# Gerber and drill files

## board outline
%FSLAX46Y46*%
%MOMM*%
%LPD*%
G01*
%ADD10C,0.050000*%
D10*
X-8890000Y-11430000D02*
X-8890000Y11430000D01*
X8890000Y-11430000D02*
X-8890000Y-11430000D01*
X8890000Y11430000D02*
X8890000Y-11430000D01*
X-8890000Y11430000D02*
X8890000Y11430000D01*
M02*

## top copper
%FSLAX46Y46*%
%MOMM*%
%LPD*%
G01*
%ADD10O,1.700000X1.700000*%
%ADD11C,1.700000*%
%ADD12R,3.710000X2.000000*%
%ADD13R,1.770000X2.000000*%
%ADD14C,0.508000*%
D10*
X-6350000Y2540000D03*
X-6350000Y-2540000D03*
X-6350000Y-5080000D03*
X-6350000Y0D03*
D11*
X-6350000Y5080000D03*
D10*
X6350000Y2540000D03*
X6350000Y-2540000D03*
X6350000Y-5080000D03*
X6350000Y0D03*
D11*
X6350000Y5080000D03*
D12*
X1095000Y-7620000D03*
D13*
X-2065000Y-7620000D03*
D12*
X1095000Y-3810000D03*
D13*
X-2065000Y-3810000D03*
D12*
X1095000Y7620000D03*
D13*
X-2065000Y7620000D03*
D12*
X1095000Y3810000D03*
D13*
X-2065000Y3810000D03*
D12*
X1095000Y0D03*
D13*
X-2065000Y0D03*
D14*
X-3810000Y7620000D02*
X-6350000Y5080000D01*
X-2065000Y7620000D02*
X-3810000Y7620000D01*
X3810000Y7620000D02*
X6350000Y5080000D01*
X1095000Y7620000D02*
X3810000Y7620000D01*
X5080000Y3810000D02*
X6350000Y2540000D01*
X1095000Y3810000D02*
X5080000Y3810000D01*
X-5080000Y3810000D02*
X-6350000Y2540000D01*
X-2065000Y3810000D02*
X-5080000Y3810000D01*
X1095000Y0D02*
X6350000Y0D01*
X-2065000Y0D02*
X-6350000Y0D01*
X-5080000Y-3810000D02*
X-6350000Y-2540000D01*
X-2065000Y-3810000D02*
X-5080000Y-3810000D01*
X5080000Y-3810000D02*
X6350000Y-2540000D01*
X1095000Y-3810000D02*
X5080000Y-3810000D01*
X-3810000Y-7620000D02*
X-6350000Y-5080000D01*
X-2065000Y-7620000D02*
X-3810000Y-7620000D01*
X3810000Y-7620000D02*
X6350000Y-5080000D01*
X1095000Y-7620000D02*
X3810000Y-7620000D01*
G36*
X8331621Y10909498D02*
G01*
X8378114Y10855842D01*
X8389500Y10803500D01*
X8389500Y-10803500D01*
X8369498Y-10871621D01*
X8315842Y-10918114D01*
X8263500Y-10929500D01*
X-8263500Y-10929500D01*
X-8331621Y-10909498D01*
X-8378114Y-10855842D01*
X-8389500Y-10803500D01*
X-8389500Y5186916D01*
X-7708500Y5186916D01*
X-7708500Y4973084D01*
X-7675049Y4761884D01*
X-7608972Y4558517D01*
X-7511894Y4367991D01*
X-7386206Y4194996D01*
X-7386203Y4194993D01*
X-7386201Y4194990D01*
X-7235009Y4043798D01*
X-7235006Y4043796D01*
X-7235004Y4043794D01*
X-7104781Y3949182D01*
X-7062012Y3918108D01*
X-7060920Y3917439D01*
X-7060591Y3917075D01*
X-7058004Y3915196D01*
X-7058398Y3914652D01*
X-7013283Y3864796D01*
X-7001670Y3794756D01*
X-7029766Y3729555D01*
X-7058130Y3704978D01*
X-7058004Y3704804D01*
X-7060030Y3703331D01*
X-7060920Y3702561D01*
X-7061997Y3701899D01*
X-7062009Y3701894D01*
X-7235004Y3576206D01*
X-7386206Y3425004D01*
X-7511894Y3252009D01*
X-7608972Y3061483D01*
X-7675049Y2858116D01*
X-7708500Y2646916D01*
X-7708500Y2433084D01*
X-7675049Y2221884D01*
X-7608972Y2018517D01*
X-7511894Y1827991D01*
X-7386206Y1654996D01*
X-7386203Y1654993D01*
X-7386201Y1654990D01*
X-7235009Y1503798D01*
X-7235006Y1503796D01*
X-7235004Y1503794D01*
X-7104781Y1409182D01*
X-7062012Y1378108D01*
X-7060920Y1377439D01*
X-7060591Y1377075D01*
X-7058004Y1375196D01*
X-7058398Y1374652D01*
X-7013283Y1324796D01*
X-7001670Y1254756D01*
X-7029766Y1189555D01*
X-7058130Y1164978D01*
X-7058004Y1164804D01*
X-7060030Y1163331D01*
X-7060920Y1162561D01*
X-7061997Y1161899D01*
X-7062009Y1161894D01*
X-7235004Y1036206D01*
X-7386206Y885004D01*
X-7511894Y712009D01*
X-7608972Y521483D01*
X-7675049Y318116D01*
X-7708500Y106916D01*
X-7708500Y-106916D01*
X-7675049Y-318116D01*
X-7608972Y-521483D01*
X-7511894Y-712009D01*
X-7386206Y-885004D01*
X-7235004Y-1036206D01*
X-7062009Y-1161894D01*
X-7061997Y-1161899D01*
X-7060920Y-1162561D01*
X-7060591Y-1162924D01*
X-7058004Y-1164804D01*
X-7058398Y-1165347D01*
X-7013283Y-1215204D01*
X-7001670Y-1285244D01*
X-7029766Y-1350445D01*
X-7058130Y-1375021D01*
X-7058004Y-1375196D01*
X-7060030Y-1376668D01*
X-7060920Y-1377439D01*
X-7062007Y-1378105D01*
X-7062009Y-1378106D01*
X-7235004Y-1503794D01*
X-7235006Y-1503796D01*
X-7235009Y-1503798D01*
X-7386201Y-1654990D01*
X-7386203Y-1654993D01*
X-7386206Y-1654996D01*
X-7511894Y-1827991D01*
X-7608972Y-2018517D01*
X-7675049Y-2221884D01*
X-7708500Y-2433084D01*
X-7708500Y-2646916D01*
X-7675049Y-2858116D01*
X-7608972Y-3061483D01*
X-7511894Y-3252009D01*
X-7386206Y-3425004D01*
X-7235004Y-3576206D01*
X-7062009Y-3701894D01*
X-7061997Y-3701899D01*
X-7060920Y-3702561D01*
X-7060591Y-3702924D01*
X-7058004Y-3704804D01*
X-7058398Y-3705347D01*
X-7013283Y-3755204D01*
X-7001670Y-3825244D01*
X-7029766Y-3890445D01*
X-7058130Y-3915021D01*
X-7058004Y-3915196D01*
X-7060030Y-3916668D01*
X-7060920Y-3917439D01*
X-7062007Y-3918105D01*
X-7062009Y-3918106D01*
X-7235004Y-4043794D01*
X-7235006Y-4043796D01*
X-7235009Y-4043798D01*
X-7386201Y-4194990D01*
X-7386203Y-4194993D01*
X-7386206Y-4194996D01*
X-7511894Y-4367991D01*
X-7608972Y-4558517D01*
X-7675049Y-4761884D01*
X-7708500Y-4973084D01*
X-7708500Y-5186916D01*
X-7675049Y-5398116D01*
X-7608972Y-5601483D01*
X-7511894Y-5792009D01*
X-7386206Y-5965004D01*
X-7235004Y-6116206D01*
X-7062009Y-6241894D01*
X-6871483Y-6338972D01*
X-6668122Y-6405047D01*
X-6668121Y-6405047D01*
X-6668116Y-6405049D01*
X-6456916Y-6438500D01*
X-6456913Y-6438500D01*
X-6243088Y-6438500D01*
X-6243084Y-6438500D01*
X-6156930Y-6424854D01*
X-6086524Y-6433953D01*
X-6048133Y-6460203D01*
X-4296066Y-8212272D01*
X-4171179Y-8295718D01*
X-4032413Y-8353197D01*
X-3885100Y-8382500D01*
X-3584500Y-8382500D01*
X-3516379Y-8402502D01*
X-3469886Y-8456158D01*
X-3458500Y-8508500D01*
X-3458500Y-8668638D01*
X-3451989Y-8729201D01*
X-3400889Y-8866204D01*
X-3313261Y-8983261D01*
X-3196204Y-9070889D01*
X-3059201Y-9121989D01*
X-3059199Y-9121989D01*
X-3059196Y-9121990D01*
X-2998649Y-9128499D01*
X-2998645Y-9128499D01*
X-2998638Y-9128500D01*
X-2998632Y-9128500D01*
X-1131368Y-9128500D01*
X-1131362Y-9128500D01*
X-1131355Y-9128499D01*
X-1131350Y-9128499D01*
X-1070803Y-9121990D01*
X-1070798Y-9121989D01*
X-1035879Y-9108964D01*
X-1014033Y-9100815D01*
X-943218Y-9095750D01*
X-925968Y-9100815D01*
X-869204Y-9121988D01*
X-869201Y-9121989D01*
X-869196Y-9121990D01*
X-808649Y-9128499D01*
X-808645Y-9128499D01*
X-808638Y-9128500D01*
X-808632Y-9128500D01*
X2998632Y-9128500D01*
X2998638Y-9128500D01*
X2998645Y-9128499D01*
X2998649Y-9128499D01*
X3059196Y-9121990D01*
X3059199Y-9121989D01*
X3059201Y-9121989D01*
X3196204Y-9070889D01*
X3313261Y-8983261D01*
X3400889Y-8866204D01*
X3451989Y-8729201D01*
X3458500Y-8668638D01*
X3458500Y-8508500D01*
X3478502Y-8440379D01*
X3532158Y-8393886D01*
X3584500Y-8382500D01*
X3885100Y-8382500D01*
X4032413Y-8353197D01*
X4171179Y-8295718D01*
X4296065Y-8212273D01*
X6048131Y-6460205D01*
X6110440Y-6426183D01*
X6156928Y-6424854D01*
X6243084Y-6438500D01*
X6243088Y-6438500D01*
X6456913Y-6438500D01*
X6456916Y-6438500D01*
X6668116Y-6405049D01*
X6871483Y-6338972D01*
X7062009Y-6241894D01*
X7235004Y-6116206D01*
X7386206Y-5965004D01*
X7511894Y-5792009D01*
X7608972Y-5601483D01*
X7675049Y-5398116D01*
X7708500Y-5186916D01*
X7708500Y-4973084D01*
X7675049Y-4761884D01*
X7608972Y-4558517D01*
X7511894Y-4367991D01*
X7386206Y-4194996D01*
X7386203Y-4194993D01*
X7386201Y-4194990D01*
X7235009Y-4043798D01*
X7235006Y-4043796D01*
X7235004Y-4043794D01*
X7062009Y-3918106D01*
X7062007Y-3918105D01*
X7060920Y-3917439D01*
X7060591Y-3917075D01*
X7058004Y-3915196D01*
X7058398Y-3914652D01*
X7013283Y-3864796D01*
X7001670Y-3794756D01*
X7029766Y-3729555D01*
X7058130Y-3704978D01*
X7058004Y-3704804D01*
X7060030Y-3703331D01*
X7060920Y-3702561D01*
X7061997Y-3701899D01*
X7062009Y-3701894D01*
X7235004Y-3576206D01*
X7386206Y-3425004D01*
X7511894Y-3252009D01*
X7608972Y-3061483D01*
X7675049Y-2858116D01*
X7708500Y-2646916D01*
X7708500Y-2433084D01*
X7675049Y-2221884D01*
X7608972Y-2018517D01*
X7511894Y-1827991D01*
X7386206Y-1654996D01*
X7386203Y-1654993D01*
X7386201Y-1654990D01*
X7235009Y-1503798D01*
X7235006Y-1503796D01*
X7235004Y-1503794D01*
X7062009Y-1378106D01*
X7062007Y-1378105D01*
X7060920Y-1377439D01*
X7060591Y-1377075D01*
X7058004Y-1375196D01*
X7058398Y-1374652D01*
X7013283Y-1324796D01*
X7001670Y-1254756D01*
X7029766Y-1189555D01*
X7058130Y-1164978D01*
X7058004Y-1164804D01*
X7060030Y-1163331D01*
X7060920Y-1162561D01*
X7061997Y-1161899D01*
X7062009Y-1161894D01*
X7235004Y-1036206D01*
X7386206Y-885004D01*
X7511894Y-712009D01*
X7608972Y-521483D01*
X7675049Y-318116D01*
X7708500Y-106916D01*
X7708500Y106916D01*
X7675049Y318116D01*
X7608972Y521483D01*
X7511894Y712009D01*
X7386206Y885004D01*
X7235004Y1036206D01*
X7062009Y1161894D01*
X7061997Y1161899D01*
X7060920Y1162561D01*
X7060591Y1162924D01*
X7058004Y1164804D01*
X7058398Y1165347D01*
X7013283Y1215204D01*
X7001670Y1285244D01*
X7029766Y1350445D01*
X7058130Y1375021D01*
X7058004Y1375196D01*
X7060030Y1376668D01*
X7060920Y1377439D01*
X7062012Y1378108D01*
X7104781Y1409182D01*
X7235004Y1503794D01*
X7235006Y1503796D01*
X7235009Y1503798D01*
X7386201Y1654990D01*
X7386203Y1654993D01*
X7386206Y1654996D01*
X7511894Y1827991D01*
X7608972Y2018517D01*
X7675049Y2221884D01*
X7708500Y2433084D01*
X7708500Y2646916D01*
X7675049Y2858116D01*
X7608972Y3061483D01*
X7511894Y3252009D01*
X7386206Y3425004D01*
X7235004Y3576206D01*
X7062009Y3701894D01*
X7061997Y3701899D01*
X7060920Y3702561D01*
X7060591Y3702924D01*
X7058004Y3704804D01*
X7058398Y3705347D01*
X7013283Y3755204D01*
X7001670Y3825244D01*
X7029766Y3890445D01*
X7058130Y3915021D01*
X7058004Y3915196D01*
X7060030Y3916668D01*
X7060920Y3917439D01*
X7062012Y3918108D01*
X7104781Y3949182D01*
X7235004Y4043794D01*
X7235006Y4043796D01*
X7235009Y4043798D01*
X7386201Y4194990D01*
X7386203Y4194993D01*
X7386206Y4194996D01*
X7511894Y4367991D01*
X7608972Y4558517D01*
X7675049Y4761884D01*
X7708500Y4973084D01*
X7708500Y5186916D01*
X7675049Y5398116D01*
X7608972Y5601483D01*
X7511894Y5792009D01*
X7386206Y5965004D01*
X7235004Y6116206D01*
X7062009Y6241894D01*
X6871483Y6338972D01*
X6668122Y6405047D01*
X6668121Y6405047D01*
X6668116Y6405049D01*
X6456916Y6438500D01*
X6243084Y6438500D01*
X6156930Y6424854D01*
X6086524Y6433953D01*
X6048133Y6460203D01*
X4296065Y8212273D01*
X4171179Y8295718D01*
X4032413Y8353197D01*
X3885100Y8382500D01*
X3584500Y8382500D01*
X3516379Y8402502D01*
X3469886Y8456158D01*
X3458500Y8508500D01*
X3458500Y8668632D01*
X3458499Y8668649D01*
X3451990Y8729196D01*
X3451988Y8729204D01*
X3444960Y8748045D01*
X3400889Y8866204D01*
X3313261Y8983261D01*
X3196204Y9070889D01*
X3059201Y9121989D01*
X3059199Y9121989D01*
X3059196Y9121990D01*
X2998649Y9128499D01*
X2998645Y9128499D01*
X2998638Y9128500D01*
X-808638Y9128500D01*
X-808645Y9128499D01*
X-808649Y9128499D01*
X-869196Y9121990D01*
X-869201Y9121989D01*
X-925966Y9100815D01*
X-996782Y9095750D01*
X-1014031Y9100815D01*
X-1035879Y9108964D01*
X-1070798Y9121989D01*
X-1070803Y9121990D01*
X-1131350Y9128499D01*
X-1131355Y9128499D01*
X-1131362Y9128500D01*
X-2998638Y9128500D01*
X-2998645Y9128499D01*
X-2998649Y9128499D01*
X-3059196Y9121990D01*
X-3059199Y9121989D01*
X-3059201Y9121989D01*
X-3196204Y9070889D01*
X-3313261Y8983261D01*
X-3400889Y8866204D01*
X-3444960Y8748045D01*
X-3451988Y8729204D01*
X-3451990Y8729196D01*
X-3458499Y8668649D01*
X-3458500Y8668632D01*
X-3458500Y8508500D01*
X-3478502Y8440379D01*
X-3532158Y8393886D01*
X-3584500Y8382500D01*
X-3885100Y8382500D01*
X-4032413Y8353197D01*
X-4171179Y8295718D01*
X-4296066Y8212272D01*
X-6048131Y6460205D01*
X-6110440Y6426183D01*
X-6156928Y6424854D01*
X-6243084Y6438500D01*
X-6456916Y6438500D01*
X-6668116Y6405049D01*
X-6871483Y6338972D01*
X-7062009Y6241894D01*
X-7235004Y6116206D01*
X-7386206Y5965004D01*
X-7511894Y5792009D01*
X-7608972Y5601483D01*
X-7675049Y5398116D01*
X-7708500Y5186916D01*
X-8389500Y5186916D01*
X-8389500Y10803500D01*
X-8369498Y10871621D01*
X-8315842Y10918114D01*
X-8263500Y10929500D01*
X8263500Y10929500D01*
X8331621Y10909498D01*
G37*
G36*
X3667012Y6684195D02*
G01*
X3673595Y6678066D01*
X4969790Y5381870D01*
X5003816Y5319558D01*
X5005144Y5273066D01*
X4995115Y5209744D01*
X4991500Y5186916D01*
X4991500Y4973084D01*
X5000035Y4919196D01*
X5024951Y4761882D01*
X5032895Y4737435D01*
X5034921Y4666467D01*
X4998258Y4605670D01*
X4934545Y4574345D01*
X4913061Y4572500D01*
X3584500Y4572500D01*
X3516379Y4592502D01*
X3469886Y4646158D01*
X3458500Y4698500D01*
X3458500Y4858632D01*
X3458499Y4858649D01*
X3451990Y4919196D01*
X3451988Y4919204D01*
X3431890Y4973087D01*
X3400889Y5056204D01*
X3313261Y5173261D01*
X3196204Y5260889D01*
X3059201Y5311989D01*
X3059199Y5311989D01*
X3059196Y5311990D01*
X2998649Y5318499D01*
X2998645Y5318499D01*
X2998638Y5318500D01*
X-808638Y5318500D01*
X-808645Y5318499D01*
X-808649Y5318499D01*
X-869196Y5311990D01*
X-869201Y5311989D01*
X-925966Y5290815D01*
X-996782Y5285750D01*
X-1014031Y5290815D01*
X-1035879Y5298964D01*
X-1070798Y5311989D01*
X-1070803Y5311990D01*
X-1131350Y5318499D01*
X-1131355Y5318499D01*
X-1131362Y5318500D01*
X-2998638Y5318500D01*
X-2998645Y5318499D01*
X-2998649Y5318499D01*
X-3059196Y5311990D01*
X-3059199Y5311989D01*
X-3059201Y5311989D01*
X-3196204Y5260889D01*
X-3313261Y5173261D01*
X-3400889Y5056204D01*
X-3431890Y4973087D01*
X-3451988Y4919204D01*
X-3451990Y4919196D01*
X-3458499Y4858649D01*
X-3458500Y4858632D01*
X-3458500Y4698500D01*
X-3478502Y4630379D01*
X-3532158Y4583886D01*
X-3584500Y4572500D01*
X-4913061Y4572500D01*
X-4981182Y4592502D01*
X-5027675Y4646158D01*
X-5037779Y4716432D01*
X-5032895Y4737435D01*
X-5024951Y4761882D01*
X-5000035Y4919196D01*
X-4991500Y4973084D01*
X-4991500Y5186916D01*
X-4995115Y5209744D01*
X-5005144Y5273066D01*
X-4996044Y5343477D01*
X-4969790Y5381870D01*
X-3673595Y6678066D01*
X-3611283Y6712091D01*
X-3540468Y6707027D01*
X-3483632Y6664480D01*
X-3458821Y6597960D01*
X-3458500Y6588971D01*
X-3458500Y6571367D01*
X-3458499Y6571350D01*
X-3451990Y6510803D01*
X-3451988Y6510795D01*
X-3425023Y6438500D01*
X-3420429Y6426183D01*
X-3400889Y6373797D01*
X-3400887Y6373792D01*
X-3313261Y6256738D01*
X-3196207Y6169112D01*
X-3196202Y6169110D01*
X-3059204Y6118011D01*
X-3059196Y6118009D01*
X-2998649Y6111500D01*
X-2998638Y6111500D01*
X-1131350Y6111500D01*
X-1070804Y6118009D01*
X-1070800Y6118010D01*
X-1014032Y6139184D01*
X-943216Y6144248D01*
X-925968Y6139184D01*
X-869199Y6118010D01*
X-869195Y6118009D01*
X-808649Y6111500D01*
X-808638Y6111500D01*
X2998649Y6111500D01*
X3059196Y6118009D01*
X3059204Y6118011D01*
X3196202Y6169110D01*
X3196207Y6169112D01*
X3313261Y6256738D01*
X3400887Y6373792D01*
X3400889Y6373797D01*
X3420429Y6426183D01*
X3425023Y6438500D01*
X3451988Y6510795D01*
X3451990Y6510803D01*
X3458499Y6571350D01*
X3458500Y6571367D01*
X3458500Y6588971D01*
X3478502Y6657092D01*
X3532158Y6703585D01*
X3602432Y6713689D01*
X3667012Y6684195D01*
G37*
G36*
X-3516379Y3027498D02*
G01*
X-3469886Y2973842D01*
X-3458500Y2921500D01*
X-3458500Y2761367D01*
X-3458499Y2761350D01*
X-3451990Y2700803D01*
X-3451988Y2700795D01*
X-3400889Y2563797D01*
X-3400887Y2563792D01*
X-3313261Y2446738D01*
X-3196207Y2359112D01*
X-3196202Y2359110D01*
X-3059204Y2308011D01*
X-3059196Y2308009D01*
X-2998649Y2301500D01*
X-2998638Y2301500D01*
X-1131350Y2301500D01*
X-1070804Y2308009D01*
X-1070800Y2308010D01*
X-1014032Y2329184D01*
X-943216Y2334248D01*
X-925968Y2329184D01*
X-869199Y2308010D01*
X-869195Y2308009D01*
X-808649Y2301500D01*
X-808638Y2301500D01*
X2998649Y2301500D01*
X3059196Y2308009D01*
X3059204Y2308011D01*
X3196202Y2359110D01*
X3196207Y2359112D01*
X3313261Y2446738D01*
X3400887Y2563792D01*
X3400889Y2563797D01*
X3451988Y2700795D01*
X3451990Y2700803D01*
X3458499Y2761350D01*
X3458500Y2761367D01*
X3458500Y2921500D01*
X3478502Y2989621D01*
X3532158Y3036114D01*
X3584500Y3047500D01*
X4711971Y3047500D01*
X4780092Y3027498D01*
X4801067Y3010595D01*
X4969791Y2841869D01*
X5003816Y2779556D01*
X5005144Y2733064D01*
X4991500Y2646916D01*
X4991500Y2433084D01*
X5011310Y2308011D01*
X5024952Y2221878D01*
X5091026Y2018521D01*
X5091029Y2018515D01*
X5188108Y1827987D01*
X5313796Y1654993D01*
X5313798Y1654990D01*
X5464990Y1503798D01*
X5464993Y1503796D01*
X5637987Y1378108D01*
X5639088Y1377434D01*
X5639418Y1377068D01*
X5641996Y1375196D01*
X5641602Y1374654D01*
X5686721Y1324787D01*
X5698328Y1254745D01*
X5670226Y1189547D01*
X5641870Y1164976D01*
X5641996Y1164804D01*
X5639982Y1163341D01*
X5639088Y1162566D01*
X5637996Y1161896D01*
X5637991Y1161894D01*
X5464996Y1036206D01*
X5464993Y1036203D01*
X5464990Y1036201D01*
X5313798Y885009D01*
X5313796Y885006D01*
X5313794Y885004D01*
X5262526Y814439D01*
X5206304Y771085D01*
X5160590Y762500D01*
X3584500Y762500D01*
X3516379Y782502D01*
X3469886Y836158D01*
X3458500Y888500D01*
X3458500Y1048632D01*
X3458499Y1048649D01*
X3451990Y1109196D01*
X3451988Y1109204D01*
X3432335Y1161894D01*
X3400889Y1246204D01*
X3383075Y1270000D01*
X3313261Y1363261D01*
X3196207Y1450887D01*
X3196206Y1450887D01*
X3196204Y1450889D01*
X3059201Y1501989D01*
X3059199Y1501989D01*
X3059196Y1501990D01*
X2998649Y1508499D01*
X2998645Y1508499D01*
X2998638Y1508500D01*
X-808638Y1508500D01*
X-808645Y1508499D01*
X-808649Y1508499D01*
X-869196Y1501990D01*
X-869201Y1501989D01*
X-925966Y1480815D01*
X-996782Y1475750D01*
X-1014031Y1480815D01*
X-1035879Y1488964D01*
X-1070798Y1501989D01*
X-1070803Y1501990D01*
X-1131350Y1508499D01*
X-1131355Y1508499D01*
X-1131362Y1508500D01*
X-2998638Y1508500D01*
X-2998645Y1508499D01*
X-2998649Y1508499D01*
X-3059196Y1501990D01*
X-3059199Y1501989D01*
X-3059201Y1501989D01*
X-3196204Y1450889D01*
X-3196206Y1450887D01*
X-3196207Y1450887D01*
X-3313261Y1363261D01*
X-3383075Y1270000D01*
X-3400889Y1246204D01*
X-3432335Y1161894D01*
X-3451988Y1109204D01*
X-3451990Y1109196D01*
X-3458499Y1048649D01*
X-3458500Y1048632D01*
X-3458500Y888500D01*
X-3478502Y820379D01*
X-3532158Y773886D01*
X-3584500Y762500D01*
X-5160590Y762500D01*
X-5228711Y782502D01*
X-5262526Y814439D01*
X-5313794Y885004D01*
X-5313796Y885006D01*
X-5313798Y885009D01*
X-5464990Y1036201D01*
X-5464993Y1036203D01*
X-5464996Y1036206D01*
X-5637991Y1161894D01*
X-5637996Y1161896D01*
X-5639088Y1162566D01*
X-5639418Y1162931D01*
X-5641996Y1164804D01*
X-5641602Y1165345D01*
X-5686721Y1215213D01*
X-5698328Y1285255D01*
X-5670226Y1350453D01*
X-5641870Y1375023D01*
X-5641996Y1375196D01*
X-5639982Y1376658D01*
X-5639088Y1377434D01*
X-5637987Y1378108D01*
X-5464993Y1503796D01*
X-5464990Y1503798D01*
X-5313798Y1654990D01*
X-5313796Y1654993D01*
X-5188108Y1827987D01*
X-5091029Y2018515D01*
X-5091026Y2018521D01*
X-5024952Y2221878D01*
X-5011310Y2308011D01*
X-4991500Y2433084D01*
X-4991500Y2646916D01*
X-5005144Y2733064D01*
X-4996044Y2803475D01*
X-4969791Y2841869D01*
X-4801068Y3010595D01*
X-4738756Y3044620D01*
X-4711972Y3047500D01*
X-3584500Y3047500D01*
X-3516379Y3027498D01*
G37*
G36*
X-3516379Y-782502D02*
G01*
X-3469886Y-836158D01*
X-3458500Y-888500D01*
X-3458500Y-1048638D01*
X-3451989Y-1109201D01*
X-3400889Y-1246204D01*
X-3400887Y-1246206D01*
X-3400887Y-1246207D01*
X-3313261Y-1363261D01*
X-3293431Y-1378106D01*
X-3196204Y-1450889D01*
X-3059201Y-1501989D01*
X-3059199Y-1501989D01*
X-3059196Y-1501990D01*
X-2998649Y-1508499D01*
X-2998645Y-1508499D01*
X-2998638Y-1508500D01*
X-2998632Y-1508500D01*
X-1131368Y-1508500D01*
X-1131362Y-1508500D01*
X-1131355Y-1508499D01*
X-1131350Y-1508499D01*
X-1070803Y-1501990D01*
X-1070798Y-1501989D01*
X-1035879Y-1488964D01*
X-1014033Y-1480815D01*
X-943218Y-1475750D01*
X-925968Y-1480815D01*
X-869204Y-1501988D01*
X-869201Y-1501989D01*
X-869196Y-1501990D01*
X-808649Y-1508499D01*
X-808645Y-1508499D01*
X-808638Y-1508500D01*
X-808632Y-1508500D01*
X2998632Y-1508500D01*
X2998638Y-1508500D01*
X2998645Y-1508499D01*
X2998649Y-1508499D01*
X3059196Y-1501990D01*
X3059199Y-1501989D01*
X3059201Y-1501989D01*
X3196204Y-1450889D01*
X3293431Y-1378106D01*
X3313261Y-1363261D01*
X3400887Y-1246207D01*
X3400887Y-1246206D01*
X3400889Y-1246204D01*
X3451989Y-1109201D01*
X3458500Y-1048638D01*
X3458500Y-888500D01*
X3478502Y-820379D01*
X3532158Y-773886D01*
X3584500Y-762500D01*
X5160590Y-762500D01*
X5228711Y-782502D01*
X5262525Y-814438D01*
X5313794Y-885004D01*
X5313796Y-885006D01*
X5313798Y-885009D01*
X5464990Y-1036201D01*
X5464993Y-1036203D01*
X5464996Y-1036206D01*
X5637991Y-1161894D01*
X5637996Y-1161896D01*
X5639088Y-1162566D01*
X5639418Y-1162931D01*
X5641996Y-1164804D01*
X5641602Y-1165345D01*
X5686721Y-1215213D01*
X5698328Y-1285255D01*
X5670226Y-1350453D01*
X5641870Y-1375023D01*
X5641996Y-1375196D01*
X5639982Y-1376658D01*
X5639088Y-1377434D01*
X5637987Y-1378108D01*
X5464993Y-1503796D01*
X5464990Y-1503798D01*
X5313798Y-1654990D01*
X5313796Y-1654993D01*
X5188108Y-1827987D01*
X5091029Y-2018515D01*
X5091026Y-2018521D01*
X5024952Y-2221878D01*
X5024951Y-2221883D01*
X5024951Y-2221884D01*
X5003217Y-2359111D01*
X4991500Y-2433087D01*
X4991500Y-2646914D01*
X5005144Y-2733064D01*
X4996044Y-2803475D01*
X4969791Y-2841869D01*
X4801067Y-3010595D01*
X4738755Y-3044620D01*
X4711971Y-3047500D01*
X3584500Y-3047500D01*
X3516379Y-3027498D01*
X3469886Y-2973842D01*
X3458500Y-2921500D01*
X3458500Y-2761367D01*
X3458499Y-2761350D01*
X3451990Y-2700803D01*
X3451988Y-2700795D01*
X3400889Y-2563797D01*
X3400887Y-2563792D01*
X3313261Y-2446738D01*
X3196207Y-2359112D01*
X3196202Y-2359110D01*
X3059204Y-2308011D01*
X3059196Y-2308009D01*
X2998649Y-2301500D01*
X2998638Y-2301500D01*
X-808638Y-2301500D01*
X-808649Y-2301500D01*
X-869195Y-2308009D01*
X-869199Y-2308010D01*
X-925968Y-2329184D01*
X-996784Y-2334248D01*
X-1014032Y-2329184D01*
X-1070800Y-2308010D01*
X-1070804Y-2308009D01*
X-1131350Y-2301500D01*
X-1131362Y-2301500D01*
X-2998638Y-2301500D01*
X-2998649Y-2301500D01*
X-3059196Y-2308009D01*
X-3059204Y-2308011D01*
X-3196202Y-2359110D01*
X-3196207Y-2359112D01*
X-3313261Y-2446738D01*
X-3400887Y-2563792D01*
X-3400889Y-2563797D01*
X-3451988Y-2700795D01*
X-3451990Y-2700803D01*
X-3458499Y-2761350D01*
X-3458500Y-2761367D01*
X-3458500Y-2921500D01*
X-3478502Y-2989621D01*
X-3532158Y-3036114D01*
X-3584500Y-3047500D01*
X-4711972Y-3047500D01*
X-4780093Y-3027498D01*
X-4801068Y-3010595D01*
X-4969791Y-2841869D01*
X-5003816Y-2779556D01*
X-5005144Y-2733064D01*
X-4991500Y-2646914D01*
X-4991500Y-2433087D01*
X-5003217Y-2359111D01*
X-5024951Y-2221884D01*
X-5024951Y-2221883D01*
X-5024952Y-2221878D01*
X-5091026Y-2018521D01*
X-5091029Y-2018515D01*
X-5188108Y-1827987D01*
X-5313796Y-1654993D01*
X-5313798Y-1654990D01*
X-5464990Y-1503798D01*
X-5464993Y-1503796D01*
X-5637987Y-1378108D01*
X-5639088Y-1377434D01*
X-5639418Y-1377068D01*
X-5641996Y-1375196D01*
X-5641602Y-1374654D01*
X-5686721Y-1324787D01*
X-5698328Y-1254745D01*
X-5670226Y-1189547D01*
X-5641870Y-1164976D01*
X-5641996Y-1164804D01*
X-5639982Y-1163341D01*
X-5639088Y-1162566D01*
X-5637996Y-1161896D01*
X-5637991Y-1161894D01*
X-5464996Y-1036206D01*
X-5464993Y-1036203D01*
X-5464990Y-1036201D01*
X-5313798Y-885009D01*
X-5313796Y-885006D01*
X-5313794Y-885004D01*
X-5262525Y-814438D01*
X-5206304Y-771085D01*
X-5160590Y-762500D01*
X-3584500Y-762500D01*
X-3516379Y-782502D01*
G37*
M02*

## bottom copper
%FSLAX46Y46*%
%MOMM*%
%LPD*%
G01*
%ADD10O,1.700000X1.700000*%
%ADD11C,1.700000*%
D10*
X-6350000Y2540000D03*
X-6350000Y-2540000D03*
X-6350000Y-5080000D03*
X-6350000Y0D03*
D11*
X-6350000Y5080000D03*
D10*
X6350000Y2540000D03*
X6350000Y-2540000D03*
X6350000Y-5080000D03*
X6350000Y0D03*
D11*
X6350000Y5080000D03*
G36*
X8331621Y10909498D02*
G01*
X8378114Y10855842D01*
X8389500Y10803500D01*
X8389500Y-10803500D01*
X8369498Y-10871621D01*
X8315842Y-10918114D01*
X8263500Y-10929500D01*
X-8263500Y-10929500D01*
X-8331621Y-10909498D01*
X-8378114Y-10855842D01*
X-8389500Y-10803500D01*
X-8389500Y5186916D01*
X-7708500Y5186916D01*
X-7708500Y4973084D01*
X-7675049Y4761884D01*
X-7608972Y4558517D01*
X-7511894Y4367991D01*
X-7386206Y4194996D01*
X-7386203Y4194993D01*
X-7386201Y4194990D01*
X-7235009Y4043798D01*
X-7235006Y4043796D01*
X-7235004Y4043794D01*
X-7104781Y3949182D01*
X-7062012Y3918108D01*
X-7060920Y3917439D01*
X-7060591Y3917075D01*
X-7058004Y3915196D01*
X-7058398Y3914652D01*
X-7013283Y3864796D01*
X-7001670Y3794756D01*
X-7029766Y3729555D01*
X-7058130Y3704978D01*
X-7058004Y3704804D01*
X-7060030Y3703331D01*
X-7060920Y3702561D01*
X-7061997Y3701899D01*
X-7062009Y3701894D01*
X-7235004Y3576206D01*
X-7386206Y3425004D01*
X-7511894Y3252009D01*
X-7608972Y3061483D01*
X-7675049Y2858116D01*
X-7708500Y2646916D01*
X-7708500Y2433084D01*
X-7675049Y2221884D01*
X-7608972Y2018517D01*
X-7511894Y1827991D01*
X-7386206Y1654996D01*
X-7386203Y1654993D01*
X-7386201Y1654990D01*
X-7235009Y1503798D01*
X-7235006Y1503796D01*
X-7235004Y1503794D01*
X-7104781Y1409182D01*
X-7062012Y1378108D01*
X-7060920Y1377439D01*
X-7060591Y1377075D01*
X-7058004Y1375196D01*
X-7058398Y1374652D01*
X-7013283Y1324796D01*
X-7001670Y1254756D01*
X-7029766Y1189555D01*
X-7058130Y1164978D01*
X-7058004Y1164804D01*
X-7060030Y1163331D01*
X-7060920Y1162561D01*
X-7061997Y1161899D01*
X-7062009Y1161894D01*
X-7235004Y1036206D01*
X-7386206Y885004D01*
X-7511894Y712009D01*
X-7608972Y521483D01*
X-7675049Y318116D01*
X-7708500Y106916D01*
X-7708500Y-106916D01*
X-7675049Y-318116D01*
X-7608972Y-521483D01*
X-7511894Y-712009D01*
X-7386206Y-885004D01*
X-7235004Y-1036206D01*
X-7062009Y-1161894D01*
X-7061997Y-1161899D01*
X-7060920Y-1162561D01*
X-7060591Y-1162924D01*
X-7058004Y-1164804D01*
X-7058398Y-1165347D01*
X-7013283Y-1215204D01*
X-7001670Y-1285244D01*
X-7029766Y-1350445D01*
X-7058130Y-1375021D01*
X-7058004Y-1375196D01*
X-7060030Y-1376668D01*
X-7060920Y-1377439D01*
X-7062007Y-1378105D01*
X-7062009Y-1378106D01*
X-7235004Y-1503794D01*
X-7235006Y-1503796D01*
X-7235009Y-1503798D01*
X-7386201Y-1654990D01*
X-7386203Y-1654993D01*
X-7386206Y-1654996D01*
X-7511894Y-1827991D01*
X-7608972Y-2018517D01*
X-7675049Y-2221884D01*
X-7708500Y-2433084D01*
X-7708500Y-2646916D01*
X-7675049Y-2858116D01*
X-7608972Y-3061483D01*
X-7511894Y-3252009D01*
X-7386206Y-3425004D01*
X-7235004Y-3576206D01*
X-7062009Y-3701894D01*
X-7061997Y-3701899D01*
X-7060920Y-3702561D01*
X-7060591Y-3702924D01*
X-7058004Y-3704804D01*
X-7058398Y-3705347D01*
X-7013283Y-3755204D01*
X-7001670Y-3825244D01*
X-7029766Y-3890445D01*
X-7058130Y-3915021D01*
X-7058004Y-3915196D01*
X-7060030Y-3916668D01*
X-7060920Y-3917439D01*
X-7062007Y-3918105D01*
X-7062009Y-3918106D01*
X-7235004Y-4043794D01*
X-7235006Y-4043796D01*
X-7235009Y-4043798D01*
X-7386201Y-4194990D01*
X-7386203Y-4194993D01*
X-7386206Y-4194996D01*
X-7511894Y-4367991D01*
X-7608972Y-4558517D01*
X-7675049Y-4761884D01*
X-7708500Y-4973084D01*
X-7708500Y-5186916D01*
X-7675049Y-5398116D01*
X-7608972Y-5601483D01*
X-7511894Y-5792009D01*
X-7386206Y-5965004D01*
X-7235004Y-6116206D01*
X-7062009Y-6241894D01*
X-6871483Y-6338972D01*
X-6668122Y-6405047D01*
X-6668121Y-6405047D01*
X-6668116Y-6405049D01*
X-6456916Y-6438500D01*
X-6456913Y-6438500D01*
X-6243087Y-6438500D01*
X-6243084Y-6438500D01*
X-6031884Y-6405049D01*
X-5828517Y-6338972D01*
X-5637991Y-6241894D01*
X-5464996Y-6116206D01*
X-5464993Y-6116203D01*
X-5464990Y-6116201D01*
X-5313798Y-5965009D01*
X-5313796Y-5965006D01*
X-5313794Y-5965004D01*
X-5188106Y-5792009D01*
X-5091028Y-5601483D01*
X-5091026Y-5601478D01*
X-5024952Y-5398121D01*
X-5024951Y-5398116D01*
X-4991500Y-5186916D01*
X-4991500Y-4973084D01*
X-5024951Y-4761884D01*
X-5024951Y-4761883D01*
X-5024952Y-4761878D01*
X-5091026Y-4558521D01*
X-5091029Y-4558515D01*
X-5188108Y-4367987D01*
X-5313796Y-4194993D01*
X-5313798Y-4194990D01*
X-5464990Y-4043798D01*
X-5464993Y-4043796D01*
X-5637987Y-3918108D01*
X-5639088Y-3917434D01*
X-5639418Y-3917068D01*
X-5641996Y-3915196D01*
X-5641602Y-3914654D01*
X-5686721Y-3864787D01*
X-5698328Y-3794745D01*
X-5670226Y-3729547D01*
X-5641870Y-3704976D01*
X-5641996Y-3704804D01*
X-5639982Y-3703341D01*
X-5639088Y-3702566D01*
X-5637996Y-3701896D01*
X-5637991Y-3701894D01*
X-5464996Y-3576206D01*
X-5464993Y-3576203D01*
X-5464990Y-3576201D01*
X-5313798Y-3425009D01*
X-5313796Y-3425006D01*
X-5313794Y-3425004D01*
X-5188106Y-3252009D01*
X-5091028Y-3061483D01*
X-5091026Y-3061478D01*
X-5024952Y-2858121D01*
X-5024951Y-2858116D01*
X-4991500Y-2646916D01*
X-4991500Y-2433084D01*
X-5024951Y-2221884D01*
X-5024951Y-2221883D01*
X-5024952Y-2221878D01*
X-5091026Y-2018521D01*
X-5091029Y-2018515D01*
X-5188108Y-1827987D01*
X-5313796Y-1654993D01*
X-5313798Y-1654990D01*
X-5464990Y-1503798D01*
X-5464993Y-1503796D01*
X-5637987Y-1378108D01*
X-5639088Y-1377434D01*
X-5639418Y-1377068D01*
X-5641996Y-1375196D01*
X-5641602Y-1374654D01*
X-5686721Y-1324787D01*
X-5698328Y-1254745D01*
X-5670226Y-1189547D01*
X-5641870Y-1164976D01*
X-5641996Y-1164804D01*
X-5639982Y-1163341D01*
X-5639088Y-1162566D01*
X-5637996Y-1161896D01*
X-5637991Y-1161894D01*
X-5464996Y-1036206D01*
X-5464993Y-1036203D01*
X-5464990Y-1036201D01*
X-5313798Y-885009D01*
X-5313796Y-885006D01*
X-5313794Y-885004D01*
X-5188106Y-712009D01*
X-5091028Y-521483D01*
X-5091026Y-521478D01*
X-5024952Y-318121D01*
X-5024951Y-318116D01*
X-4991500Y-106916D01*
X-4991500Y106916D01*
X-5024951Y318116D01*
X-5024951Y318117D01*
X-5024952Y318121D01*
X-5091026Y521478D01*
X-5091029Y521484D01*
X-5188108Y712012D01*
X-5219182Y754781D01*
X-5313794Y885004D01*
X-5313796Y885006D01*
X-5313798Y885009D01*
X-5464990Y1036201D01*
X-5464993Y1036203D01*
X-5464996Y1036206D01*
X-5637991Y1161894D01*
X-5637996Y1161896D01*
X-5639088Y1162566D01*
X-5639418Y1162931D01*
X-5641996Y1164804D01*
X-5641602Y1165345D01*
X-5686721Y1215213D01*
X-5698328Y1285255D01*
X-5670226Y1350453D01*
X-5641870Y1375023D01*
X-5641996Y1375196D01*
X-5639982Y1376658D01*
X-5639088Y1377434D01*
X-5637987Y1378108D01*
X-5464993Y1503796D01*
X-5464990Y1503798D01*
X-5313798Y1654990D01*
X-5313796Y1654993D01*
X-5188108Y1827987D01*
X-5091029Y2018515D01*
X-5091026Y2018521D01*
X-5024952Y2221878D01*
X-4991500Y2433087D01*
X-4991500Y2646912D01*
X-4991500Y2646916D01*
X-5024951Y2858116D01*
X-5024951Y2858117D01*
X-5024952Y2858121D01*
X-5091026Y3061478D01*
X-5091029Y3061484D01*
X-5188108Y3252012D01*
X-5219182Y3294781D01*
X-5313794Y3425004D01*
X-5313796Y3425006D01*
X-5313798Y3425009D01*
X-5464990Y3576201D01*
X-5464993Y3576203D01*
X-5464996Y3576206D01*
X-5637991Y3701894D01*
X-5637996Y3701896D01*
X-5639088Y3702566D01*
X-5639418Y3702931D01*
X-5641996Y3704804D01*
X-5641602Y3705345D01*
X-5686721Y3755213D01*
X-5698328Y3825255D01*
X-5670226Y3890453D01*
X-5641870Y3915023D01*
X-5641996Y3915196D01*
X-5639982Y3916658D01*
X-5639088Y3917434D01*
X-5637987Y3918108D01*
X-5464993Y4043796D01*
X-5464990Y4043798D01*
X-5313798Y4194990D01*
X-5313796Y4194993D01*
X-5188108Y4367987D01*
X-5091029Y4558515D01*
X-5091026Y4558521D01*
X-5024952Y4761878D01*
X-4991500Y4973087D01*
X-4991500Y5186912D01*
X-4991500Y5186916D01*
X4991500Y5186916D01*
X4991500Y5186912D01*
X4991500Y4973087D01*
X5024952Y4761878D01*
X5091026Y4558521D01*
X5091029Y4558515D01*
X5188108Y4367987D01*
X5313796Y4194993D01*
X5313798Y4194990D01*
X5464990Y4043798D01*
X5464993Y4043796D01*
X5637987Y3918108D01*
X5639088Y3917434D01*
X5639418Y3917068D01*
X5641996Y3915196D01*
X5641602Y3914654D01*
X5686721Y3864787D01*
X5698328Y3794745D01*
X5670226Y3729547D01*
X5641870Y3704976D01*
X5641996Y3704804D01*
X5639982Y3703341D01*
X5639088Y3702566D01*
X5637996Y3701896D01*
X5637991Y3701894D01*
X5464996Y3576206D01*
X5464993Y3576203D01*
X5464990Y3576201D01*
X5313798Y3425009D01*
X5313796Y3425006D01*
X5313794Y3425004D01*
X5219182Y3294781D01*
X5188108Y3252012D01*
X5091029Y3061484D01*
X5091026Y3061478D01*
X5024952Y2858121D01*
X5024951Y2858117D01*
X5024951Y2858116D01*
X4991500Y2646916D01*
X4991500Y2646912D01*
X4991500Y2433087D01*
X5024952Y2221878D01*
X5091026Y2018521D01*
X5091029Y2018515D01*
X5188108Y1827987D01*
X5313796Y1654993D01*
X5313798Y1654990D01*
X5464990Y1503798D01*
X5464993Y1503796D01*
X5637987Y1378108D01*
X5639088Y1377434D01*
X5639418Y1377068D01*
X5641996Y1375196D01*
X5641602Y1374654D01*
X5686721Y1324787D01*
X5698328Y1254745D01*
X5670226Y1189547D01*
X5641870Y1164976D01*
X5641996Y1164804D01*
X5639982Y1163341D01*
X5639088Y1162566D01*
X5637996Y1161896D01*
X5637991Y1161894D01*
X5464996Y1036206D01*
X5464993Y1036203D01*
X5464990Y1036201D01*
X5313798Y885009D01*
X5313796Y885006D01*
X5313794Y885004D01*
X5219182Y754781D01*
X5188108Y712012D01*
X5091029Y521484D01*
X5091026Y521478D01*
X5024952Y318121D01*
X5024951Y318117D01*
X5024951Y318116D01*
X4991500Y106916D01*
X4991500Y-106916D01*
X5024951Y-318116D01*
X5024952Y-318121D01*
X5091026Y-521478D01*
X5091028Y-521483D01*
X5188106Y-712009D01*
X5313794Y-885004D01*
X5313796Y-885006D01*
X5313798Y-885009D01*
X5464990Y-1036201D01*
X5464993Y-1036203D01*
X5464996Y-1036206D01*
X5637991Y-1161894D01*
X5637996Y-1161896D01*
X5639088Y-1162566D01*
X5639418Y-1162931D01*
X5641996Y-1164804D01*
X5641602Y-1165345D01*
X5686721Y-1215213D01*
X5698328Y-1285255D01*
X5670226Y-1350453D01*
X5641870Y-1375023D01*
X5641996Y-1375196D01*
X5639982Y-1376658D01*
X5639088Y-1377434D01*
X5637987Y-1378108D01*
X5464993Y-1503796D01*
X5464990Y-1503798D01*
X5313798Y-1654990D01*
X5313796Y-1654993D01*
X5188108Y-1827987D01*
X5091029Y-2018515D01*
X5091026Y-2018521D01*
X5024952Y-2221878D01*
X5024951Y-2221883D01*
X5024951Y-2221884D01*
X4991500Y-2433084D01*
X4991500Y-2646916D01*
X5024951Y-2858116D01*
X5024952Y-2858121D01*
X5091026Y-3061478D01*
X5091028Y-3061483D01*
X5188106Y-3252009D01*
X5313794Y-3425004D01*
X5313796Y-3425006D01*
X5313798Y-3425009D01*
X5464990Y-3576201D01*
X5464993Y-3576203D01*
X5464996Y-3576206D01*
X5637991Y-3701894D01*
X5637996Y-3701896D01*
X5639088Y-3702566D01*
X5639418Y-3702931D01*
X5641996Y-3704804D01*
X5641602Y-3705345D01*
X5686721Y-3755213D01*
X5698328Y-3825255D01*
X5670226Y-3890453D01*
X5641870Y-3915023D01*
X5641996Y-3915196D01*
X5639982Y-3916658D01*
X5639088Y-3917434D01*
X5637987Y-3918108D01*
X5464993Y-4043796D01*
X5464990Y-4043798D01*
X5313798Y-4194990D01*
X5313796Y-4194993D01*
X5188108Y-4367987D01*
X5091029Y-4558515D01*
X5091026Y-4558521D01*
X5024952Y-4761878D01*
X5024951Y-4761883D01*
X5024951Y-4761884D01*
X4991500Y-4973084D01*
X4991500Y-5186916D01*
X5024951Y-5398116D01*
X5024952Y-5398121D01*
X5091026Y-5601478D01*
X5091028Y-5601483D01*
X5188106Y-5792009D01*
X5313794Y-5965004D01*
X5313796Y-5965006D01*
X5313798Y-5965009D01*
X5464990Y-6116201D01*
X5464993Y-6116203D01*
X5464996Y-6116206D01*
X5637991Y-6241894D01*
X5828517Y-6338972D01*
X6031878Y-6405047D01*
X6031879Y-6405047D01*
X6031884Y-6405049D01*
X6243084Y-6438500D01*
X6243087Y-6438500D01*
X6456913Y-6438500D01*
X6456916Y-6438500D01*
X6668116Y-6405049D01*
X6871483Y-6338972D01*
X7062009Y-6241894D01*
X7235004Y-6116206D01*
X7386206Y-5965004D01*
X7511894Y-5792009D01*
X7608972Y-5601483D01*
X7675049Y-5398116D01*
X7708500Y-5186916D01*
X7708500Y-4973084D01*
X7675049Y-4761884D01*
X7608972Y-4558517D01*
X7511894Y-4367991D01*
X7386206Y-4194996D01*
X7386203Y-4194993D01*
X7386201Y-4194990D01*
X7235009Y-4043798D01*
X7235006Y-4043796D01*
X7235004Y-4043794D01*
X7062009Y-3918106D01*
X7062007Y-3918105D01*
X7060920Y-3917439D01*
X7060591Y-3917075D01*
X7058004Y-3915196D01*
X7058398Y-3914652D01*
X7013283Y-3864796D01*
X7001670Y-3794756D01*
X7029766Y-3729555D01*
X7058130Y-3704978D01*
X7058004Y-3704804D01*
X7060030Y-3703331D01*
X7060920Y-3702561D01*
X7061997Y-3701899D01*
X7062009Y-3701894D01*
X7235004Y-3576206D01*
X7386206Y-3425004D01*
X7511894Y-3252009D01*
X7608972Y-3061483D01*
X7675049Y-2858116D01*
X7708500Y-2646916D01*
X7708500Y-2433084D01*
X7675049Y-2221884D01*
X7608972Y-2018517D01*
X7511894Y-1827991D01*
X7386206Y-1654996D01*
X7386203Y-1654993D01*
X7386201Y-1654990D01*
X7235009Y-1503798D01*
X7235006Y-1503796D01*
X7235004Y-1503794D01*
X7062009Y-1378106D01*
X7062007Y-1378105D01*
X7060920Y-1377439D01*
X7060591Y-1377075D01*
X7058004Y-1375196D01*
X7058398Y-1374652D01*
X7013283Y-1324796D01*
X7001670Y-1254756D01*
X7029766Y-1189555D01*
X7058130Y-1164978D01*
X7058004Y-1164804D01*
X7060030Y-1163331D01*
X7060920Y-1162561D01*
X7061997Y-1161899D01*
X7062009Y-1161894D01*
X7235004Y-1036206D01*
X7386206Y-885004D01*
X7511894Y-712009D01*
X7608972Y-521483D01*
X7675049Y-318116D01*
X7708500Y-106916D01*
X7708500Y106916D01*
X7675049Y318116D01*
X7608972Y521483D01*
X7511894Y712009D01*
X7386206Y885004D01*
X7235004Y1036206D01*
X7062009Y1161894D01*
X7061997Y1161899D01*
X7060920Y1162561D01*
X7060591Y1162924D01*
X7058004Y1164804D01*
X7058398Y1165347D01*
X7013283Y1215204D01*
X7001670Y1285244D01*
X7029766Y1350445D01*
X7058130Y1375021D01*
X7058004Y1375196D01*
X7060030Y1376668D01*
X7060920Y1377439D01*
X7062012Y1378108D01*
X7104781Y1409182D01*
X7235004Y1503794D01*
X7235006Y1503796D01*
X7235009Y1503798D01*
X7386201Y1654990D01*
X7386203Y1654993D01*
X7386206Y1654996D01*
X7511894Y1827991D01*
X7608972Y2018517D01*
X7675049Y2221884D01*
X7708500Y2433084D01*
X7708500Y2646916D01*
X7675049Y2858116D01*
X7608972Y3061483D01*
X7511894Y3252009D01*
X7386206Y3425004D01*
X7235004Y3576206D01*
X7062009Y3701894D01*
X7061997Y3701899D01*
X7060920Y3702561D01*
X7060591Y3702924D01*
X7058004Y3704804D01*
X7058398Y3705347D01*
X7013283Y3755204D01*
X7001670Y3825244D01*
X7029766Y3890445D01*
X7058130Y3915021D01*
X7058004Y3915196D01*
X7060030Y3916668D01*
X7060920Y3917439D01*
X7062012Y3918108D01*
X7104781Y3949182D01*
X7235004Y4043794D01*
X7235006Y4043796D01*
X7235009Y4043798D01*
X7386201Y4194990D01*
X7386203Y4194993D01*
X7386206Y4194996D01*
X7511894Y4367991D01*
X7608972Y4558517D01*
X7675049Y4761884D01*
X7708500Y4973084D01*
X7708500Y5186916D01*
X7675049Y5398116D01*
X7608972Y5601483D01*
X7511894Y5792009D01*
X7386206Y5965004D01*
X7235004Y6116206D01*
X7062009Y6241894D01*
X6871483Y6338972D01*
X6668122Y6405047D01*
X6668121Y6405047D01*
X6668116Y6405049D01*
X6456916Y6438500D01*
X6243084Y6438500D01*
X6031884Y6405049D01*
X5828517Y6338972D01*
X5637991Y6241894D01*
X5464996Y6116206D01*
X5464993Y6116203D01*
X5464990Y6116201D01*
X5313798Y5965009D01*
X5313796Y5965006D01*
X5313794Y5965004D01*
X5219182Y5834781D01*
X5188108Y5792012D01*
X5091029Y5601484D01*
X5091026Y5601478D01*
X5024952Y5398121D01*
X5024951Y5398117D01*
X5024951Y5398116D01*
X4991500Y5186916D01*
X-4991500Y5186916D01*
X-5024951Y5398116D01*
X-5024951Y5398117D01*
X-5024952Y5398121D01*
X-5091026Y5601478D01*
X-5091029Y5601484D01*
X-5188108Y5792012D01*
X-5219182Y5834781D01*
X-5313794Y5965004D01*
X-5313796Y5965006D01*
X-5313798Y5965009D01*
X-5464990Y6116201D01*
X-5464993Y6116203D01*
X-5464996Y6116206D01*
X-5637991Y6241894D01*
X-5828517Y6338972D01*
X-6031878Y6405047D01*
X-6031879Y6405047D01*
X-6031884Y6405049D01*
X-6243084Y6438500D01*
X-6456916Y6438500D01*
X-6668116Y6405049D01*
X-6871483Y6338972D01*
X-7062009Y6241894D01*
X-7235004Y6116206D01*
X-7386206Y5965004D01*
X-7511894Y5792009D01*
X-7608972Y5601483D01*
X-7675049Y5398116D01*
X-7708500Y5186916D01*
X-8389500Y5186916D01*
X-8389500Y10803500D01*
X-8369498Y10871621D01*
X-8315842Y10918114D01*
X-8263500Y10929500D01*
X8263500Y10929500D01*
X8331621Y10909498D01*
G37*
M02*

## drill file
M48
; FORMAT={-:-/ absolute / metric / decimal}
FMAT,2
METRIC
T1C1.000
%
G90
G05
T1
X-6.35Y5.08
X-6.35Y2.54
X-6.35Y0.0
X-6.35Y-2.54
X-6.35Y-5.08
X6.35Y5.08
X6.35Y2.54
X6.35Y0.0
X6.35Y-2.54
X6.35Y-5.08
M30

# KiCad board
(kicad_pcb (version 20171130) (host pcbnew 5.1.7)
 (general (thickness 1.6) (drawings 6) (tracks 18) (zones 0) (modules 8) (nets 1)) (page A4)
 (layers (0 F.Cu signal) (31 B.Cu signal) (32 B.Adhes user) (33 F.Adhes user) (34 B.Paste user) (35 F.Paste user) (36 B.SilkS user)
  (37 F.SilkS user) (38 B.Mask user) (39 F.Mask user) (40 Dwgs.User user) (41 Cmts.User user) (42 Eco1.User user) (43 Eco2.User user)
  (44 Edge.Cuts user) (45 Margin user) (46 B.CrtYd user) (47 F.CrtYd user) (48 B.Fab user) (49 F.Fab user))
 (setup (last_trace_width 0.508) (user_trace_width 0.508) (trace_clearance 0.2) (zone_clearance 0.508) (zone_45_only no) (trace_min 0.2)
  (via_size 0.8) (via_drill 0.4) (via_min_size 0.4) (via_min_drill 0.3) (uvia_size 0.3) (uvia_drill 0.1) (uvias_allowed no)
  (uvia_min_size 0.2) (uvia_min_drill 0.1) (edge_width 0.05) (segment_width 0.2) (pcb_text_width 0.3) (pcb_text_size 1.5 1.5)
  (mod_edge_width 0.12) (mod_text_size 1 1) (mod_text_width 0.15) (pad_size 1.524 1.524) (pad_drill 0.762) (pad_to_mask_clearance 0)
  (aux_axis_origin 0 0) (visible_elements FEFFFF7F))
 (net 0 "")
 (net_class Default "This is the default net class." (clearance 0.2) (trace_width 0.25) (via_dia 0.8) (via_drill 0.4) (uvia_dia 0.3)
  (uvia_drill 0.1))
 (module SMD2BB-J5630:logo (layer B.Cu) (at 0 0 180)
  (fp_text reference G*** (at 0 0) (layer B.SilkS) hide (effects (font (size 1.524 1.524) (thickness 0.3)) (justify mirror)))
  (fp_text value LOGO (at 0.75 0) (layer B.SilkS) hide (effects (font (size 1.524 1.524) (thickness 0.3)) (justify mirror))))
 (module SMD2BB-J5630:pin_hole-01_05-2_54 (layer F.Cu) (at -6.35 0)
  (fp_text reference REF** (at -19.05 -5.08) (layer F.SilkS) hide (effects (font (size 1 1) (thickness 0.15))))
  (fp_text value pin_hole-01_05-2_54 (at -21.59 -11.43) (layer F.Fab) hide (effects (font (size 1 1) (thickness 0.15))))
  (pad 2 thru_hole oval (at 0 -2.54) (size 1.7 1.7) (drill 1) (layers *.Cu *.Mask))
  (pad 4 thru_hole oval (at 0 2.54) (size 1.7 1.7) (drill 1) (layers *.Cu *.Mask))
  (pad 5 thru_hole oval (at 0 5.08) (size 1.7 1.7) (drill 1) (layers *.Cu *.Mask))
  (pad 3 thru_hole oval (at 0 0) (size 1.7 1.7) (drill 1) (layers *.Cu *.Mask))
  (pad 1 thru_hole circle (at 0 -5.08) (size 1.7 1.7) (drill 1) (layers *.Cu *.Mask)))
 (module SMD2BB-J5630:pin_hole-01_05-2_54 (layer F.Cu) (at 6.35 0)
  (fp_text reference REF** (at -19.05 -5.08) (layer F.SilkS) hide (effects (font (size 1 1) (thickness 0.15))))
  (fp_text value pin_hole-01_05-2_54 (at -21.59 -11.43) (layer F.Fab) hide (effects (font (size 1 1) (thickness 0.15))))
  (pad 2 thru_hole oval (at 0 -2.54) (size 1.7 1.7) (drill 1) (layers *.Cu *.Mask))
  (pad 4 thru_hole oval (at 0 2.54) (size 1.7 1.7) (drill 1) (layers *.Cu *.Mask))
  (pad 5 thru_hole oval (at 0 5.08) (size 1.7 1.7) (drill 1) (layers *.Cu *.Mask))
  (pad 3 thru_hole oval (at 0 0) (size 1.7 1.7) (drill 1) (layers *.Cu *.Mask))
  (pad 1 thru_hole circle (at 0 -5.08) (size 1.7 1.7) (drill 1) (layers *.Cu *.Mask)))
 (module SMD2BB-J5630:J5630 (layer F.Cu) (at 0 7.62)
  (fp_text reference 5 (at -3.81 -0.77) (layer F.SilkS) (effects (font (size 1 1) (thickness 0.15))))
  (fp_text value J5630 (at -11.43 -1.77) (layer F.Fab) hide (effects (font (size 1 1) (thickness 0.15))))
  (pad 2 smd rect (at 1.095 0) (size 3.71 2) (layers F.Cu F.Paste F.Mask))
  (pad 1 smd rect (at -2.065 0) (size 1.77 2) (layers F.Cu F.Paste F.Mask)))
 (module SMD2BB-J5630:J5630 (layer F.Cu) (at 0 3.81)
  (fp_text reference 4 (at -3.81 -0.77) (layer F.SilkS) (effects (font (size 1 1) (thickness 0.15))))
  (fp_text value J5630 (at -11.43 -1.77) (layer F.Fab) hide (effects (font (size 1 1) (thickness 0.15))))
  (pad 2 smd rect (at 1.095 0) (size 3.71 2) (layers F.Cu F.Paste F.Mask))
  (pad 1 smd rect (at -2.065 0) (size 1.77 2) (layers F.Cu F.Paste F.Mask)))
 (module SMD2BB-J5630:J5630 (layer F.Cu) (at 0 -7.62)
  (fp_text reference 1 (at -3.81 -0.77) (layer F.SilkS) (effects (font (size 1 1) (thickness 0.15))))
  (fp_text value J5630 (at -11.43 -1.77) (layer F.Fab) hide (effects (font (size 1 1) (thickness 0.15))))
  (pad 2 smd rect (at 1.095 0) (size 3.71 2) (layers F.Cu F.Paste F.Mask))
  (pad 1 smd rect (at -2.065 0) (size 1.77 2) (layers F.Cu F.Paste F.Mask)))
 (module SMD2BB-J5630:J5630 (layer F.Cu) (at 0 -3.81)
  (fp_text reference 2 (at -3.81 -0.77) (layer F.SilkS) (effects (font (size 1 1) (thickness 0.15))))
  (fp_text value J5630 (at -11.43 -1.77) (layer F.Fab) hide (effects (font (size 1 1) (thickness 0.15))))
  (pad 2 smd rect (at 1.095 0) (size 3.71 2) (layers F.Cu F.Paste F.Mask))
  (pad 1 smd rect (at -2.065 0) (size 1.77 2) (layers F.Cu F.Paste F.Mask)))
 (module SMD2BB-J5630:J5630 (layer F.Cu) (at 0 0)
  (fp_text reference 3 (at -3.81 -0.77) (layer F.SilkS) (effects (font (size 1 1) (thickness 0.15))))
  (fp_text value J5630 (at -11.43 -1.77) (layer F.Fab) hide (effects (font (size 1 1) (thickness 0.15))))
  (pad 2 smd rect (at 1.095 0) (size 3.71 2) (layers F.Cu F.Paste F.Mask))
  (pad 1 smd rect (at -2.065 0) (size 1.77 2) (layers F.Cu F.Paste F.Mask)))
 (gr_line (start -8.89 11.43) (end -8.89 -11.43) (layer Edge.Cuts) (width 0.05))
 (gr_line (start 8.89 11.43) (end -8.89 11.43) (layer Edge.Cuts) (width 0.05))
 (gr_line (start 8.89 -11.43) (end 8.89 11.43) (layer Edge.Cuts) (width 0.05))
 (gr_line (start -8.89 -11.43) (end 8.89 -11.43) (layer Edge.Cuts) (width 0.05))
 (segment (start -3.81 -7.62) (end -6.35 -5.08) (width 0.508) (layer F.Cu) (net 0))
 (segment (start -2.065 -7.62) (end -3.81 -7.62) (width 0.508) (layer F.Cu) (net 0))
 (segment (start 3.81 -7.62) (end 6.35 -5.08) (width 0.508) (layer F.Cu) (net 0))
 (segment (start 1.095 -7.62) (end 3.81 -7.62) (width 0.508) (layer F.Cu) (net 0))
 (segment (start 5.08 -3.81) (end 6.35 -2.54) (width 0.508) (layer F.Cu) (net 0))
 (segment (start 1.095 -3.81) (end 5.08 -3.81) (width 0.508) (layer F.Cu) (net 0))
 (segment (start -5.08 -3.81) (end -6.35 -2.54) (width 0.508) (layer F.Cu) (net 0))
 (segment (start -2.065 -3.81) (end -5.08 -3.81) (width 0.508) (layer F.Cu) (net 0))
 (segment (start 1.095 0) (end 6.35 0) (width 0.508) (layer F.Cu) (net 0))
 (segment (start -2.065 0) (end -6.35 0) (width 0.508) (layer F.Cu) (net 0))
 (segment (start -5.08 3.81) (end -6.35 2.54) (width 0.508) (layer F.Cu) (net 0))
 (segment (start -2.065 3.81) (end -5.08 3.81) (width 0.508) (layer F.Cu) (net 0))
 (segment (start 5.08 3.81) (end 6.35 2.54) (width 0.508) (layer F.Cu) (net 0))
 (segment (start 1.095 3.81) (end 5.08 3.81) (width 0.508) (layer F.Cu) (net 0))
 (segment (start -3.81 7.62) (end -6.35 5.08) (width 0.508) (layer F.Cu) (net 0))
 (segment (start -2.065 7.62) (end -3.81 7.62) (width 0.508) (layer F.Cu) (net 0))
 (segment (start 3.81 7.62) (end 6.35 5.08) (width 0.508) (layer F.Cu) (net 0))
 (segment (start 1.095 7.62) (end 3.81 7.62) (width 0.508) (layer F.Cu) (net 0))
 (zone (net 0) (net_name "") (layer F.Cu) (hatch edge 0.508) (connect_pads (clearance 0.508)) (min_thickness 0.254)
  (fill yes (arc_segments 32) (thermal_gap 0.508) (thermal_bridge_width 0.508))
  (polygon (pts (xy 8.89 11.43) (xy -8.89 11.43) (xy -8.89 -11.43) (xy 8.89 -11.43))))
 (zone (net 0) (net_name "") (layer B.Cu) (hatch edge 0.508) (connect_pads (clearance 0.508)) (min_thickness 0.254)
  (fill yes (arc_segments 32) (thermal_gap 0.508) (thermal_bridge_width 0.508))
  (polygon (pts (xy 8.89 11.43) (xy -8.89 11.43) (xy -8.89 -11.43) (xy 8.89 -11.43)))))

